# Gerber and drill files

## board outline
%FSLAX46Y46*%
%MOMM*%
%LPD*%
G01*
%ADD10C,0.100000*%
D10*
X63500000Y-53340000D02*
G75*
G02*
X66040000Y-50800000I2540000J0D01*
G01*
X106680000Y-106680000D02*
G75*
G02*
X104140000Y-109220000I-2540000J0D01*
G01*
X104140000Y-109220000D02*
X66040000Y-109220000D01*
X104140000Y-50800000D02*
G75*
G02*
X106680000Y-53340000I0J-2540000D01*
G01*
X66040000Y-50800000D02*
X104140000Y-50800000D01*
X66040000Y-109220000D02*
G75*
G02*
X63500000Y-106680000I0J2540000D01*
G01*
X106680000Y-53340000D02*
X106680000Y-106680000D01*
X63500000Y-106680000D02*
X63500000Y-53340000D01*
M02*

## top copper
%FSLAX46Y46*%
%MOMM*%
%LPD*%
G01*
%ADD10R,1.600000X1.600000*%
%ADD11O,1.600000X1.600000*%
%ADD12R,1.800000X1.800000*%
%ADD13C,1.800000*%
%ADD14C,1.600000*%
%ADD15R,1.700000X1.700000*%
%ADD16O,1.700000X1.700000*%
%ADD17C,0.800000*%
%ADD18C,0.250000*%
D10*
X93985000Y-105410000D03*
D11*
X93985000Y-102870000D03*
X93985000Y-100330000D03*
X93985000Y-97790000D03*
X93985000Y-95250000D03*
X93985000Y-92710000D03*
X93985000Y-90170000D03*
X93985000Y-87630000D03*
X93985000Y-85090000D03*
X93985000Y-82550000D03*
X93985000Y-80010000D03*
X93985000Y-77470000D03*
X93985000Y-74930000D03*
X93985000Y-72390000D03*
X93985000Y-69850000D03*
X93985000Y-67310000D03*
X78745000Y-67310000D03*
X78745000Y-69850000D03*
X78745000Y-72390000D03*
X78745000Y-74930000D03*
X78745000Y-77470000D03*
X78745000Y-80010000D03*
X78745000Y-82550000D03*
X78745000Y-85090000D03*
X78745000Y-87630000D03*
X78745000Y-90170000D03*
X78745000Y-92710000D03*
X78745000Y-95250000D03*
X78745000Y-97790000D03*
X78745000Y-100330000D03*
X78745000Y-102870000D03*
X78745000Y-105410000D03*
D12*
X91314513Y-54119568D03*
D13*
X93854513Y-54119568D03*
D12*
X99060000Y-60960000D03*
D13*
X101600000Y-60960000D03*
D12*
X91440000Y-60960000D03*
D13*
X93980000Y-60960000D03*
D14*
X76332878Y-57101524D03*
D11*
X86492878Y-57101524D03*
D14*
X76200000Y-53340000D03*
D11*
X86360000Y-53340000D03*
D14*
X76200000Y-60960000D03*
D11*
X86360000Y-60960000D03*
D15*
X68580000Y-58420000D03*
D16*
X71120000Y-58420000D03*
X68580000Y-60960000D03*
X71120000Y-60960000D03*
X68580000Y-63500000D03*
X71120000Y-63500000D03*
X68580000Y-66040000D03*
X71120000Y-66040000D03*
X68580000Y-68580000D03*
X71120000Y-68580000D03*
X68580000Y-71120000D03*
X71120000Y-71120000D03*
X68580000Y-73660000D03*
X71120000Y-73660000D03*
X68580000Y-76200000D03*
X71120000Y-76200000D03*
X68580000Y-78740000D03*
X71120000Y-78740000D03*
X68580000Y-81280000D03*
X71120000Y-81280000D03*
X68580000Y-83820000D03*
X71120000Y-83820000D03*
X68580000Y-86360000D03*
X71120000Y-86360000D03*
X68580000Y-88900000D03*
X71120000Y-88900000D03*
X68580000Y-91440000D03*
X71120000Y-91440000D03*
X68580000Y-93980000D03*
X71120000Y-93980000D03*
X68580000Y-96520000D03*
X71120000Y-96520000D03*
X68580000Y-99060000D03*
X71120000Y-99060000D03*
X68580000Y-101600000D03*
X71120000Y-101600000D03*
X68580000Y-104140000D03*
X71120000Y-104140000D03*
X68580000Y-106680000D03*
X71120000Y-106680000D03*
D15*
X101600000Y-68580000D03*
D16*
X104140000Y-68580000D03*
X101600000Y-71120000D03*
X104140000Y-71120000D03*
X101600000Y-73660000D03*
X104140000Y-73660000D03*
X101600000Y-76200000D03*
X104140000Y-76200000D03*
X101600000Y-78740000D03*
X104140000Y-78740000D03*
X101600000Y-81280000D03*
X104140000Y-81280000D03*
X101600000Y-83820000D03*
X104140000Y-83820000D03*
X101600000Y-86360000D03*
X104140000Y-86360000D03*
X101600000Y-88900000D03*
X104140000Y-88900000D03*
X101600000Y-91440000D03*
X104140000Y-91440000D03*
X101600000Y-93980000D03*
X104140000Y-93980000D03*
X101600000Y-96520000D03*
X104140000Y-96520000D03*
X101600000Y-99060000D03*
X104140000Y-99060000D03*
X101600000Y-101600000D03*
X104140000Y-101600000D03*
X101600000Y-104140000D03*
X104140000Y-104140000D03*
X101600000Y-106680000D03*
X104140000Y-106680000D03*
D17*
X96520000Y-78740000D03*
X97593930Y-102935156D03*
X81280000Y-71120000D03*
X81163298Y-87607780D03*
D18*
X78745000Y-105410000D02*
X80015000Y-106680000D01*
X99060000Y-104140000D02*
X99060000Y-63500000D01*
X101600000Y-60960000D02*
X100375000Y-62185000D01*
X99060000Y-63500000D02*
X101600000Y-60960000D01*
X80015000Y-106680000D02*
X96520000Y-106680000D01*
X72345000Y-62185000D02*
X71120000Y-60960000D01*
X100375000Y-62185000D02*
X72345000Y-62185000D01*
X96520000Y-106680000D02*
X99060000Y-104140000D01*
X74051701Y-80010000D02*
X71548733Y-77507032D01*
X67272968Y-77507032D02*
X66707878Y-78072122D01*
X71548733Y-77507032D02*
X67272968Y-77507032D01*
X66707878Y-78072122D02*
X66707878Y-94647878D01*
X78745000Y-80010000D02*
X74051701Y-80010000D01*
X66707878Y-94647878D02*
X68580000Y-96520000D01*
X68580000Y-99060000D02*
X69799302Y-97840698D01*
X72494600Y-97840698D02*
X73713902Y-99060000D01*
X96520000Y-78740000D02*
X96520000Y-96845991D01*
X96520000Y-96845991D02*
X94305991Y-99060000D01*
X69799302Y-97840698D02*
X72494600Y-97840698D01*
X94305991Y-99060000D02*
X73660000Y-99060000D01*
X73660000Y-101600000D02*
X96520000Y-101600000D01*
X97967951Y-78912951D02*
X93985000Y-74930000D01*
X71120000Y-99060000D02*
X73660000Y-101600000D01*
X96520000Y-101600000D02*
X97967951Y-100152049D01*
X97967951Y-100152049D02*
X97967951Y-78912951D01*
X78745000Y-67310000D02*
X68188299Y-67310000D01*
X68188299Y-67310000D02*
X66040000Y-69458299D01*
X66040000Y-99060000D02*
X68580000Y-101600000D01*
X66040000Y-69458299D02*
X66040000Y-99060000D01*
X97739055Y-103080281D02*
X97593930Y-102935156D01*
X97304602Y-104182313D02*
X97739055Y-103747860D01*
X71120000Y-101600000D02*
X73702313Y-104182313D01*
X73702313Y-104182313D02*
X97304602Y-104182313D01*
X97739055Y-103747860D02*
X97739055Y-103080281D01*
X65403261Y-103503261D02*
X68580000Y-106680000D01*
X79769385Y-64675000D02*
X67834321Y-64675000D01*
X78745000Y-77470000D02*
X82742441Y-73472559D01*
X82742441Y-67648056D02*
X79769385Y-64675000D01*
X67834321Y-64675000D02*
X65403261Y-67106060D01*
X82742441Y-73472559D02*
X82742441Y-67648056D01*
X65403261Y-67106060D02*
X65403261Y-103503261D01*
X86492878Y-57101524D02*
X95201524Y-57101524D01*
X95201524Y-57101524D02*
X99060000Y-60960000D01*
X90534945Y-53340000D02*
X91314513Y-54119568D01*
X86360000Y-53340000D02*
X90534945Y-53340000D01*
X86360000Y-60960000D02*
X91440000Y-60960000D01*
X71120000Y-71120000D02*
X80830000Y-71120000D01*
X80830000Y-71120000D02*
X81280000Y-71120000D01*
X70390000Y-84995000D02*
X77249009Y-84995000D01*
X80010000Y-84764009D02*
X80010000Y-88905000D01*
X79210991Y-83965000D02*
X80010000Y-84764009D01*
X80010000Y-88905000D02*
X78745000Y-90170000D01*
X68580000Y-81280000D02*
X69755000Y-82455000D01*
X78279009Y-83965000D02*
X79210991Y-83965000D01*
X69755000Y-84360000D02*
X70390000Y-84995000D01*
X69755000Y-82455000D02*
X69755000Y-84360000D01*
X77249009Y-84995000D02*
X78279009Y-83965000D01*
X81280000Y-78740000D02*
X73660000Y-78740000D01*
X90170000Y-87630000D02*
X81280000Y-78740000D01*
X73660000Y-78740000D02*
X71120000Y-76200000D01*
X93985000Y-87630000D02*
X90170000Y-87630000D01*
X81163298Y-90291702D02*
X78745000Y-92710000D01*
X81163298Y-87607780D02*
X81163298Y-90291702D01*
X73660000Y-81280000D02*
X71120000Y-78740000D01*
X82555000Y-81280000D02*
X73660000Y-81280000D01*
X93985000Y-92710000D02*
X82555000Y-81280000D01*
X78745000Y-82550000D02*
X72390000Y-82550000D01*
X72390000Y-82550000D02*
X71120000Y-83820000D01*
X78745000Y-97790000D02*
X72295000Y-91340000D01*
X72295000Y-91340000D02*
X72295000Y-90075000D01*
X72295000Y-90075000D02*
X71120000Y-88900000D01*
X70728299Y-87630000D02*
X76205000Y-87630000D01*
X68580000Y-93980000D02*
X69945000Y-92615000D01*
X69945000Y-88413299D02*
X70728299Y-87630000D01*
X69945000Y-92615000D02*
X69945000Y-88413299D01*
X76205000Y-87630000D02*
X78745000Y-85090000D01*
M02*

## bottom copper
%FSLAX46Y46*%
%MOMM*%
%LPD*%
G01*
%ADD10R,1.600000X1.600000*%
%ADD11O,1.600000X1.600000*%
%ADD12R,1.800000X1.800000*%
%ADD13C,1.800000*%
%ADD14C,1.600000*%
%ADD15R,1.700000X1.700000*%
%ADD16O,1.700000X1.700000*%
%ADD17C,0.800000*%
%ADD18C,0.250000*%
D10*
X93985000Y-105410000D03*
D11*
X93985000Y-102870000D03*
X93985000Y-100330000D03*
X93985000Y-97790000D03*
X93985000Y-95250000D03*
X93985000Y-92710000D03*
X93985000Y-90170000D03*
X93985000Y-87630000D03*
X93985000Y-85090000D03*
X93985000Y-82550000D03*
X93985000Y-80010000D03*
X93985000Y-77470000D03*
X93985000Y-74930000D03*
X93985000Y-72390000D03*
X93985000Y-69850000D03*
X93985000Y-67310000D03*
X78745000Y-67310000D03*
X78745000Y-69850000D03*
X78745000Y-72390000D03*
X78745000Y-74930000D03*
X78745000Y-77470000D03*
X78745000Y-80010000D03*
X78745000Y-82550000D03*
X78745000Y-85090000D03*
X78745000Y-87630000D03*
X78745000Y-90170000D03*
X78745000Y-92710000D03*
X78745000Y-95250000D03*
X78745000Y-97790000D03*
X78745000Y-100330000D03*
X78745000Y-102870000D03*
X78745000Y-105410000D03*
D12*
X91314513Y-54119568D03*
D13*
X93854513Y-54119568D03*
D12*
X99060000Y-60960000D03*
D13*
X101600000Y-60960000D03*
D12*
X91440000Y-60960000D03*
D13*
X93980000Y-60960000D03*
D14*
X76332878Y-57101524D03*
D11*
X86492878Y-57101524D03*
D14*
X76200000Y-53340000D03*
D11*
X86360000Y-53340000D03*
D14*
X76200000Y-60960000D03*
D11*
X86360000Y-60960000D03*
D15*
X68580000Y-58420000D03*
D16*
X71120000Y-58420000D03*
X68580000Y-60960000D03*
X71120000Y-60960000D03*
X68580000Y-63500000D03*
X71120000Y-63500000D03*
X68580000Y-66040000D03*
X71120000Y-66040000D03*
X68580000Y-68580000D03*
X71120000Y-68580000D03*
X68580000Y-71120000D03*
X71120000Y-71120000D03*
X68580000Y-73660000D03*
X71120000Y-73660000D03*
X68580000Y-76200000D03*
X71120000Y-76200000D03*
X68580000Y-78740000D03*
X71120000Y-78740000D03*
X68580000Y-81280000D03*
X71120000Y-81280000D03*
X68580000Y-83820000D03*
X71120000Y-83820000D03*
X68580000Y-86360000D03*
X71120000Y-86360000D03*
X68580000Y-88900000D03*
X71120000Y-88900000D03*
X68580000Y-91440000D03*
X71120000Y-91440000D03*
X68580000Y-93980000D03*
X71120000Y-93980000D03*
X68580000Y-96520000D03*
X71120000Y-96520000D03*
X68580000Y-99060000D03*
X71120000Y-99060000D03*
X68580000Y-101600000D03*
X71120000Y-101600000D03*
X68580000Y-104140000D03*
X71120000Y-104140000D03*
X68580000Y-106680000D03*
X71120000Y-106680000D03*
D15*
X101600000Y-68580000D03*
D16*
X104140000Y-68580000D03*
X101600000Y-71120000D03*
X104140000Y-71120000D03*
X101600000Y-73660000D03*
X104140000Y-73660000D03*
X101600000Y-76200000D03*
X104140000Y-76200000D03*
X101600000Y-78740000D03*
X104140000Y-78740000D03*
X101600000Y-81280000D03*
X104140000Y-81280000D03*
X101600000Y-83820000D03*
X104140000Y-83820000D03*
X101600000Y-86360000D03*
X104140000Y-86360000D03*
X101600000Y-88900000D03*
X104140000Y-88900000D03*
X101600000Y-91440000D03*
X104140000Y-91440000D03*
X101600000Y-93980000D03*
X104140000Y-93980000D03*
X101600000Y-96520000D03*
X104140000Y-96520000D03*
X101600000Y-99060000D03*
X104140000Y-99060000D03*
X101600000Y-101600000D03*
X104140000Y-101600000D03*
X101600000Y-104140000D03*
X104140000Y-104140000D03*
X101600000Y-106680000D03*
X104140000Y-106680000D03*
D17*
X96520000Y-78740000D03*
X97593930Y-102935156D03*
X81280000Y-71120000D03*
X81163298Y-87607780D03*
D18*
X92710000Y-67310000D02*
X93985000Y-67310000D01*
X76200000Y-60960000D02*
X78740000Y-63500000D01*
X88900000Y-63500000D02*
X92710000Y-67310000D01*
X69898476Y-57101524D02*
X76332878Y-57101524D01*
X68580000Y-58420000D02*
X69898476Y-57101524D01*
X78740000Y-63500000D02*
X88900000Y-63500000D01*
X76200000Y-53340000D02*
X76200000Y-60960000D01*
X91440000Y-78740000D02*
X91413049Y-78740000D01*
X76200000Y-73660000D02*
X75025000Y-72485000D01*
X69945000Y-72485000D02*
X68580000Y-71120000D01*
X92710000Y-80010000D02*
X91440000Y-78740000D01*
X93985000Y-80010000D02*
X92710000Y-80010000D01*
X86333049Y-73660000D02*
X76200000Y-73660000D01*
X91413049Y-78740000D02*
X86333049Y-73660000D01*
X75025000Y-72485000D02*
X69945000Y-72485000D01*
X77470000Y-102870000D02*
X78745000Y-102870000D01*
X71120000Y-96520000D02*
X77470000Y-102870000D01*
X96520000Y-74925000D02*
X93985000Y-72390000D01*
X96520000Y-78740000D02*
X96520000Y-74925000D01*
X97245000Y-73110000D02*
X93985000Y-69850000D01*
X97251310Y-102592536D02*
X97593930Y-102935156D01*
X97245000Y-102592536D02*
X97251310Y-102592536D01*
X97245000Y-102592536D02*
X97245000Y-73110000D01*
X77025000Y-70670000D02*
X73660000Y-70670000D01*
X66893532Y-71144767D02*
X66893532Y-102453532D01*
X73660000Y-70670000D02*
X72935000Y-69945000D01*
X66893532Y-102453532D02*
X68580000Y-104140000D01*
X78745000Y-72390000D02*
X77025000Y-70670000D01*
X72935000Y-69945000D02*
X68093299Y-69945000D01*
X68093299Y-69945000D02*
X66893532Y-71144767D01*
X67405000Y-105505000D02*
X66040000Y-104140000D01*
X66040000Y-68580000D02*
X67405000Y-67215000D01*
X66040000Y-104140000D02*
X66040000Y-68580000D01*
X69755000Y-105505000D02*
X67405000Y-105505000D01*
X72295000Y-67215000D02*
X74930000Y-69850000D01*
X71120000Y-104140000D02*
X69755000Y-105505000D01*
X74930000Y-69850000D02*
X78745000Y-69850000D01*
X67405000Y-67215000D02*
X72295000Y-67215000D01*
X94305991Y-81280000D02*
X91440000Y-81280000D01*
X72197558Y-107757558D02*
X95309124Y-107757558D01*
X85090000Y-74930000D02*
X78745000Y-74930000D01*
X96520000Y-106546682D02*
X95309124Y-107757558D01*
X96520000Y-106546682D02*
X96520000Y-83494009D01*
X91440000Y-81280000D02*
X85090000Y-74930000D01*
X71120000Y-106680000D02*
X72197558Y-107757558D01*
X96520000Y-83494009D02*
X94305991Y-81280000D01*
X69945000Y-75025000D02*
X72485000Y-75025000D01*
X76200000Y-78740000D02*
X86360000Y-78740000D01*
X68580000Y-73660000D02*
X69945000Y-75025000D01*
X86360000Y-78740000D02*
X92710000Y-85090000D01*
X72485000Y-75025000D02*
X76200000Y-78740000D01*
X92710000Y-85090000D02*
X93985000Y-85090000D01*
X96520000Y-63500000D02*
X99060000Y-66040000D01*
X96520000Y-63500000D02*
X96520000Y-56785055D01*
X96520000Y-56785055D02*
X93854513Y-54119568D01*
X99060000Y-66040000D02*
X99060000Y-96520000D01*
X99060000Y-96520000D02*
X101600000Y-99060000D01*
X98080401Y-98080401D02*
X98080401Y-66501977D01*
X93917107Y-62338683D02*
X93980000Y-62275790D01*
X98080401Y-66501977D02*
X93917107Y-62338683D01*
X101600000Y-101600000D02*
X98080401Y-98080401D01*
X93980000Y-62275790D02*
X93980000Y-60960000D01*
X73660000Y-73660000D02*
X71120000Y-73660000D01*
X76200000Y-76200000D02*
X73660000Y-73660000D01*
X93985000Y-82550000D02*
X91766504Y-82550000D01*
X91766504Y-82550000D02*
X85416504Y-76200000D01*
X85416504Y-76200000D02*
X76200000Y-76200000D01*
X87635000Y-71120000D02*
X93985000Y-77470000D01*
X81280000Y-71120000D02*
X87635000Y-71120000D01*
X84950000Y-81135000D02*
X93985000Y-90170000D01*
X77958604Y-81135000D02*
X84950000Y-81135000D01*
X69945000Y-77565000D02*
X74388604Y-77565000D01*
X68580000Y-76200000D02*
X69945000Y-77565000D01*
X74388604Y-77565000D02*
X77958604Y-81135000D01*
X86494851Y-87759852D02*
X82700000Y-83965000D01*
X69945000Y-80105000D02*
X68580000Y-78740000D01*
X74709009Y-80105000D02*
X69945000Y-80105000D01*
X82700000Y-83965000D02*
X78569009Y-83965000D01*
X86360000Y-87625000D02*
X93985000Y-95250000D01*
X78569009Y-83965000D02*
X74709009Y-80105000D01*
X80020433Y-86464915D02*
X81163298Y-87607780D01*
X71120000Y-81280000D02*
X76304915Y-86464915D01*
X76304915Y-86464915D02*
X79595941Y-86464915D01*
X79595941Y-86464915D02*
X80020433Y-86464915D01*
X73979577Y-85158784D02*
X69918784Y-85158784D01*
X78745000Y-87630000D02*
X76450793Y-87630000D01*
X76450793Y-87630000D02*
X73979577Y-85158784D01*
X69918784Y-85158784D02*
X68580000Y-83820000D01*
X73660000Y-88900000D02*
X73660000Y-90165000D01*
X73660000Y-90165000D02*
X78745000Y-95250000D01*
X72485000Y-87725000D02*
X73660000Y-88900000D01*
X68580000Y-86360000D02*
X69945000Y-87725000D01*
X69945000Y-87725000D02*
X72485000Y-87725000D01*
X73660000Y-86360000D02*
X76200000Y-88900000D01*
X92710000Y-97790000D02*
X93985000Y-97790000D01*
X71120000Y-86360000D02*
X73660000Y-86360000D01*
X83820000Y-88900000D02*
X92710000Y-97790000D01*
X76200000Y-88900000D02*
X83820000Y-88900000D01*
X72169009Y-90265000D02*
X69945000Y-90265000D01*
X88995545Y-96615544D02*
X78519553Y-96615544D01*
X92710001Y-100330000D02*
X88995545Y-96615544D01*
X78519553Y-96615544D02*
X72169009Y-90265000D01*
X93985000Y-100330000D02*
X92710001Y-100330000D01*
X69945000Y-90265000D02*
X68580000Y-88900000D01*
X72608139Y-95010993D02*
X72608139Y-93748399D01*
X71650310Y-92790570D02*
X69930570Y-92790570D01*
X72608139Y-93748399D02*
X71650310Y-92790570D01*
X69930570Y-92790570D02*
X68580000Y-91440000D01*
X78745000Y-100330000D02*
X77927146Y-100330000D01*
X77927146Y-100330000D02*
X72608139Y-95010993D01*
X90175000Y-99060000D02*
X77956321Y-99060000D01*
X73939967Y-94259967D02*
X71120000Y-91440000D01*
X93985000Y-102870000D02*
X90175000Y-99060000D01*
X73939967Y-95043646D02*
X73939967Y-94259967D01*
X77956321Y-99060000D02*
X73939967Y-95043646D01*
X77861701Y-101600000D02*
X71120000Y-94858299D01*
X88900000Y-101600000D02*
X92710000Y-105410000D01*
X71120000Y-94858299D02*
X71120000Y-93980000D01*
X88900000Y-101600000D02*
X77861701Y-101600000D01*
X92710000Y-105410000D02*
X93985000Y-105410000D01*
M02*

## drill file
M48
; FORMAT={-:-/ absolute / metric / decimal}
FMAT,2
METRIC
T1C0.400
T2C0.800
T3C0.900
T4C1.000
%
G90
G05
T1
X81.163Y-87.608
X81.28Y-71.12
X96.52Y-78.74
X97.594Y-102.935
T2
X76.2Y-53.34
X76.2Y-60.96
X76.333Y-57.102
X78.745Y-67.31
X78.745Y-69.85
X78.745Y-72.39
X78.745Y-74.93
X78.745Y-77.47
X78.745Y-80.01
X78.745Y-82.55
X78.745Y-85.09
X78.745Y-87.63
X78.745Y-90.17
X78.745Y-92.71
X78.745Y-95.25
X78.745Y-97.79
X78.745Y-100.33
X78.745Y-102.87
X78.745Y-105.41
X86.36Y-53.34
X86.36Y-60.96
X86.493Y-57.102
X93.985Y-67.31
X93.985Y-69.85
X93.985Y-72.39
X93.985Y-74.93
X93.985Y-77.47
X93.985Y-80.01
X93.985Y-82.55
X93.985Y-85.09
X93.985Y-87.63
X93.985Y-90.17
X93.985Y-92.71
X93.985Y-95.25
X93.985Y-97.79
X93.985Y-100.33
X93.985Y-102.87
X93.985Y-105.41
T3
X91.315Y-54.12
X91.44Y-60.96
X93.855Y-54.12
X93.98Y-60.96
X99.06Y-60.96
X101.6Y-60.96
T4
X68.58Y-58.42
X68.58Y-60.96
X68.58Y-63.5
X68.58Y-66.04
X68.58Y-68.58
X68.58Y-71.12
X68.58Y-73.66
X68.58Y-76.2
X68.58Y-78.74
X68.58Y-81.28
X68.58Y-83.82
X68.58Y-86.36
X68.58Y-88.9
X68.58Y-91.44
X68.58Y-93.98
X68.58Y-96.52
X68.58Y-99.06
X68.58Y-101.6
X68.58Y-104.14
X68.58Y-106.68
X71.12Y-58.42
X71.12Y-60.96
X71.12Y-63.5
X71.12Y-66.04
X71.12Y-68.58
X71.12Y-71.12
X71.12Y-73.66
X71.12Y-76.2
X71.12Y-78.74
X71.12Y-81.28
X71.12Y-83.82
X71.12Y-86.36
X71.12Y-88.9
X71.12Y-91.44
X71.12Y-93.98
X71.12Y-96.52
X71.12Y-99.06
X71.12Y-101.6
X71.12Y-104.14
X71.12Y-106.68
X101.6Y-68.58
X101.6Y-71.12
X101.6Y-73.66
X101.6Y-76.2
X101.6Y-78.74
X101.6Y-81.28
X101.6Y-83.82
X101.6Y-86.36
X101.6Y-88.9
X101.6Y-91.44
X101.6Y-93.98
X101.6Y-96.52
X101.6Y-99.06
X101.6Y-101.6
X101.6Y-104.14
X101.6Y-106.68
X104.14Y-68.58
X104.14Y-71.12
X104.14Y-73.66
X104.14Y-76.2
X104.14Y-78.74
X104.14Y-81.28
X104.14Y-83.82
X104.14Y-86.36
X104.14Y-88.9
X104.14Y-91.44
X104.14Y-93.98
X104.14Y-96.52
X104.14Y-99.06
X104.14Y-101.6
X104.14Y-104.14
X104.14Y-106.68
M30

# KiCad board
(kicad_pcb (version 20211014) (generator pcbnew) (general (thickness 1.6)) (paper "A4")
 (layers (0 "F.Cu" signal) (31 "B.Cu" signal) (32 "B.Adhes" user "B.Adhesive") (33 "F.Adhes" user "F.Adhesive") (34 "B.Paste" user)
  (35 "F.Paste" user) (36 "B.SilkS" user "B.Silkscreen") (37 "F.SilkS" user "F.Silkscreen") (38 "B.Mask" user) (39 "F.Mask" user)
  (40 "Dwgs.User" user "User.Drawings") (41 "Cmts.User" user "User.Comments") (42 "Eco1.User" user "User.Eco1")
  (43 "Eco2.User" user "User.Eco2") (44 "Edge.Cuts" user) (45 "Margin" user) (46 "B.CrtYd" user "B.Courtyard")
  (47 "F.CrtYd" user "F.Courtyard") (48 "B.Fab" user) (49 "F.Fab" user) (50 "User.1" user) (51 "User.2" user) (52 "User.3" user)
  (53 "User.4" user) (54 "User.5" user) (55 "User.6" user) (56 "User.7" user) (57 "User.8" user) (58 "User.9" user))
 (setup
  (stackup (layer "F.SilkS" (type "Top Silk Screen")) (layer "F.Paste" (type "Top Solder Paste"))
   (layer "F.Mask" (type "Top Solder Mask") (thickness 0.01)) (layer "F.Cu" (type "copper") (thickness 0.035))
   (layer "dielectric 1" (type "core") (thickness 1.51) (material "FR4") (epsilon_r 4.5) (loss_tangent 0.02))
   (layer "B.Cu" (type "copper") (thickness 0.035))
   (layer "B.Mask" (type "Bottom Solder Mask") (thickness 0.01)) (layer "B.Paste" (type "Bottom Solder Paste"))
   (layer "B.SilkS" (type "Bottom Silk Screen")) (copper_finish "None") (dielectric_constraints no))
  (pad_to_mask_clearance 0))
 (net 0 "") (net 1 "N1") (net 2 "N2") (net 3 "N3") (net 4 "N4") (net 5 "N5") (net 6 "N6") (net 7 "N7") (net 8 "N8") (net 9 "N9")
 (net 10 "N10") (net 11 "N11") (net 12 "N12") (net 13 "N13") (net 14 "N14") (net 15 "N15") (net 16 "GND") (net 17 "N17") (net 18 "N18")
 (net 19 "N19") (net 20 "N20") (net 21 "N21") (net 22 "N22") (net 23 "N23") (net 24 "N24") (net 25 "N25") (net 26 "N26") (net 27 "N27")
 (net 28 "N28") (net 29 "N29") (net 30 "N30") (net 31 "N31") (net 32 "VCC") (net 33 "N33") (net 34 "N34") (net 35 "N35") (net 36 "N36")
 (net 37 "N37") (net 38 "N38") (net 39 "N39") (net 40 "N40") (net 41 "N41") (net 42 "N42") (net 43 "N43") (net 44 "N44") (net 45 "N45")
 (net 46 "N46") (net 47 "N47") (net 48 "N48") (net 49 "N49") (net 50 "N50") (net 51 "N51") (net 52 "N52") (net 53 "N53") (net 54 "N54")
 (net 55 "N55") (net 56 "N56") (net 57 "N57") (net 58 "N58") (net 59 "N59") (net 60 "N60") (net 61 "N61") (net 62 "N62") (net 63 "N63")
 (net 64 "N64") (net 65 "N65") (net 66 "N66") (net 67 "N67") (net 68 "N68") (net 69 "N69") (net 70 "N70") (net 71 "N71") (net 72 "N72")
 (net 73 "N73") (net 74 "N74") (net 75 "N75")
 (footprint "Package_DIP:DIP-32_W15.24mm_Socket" (layer "F.Cu") (at 93.985 105.41 180)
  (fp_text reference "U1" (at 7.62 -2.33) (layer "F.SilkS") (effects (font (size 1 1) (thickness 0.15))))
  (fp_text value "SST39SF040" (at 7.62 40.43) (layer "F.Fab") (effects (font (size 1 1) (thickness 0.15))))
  (pad "1" thru_hole rect (at 0 0 180) (size 1.6 1.6) (drill 0.8) (layers *.Cu *.Mask) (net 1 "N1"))
  (pad "2" thru_hole oval (at 0 2.54 180) (size 1.6 1.6) (drill 0.8) (layers *.Cu *.Mask) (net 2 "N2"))
  (pad "3" thru_hole oval (at 0 5.08 180) (size 1.6 1.6) (drill 0.8) (layers *.Cu *.Mask) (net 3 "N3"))
  (pad "4" thru_hole oval (at 0 7.62 180) (size 1.6 1.6) (drill 0.8) (layers *.Cu *.Mask) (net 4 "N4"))
  (pad "5" thru_hole oval (at 0 10.16 180) (size 1.6 1.6) (drill 0.8) (layers *.Cu *.Mask) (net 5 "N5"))
  (pad "6" thru_hole oval (at 0 12.7 180) (size 1.6 1.6) (drill 0.8) (layers *.Cu *.Mask) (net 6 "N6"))
  (pad "7" thru_hole oval (at 0 15.24 180) (size 1.6 1.6) (drill 0.8) (layers *.Cu *.Mask) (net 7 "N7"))
  (pad "8" thru_hole oval (at 0 17.78 180) (size 1.6 1.6) (drill 0.8) (layers *.Cu *.Mask) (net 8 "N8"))
  (pad "9" thru_hole oval (at 0 20.32 180) (size 1.6 1.6) (drill 0.8) (layers *.Cu *.Mask) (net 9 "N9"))
  (pad "10" thru_hole oval (at 0 22.86 180) (size 1.6 1.6) (drill 0.8) (layers *.Cu *.Mask) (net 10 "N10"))
  (pad "11" thru_hole oval (at 0 25.4 180) (size 1.6 1.6) (drill 0.8) (layers *.Cu *.Mask) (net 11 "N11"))
  (pad "12" thru_hole oval (at 0 27.94 180) (size 1.6 1.6) (drill 0.8) (layers *.Cu *.Mask) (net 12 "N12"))
  (pad "13" thru_hole oval (at 0 30.48 180) (size 1.6 1.6) (drill 0.8) (layers *.Cu *.Mask) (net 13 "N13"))
  (pad "14" thru_hole oval (at 0 33.02 180) (size 1.6 1.6) (drill 0.8) (layers *.Cu *.Mask) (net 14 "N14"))
  (pad "15" thru_hole oval (at 0 35.56 180) (size 1.6 1.6) (drill 0.8) (layers *.Cu *.Mask) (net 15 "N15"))
  (pad "16" thru_hole oval (at 0 38.1 180) (size 1.6 1.6) (drill 0.8) (layers *.Cu *.Mask) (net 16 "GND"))
  (pad "17" thru_hole oval (at 15.24 38.1 180) (size 1.6 1.6) (drill 0.8) (layers *.Cu *.Mask) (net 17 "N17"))
  (pad "18" thru_hole oval (at 15.24 35.56 180) (size 1.6 1.6) (drill 0.8) (layers *.Cu *.Mask) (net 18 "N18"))
  (pad "19" thru_hole oval (at 15.24 33.02 180) (size 1.6 1.6) (drill 0.8) (layers *.Cu *.Mask) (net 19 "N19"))
  (pad "20" thru_hole oval (at 15.24 30.48 180) (size 1.6 1.6) (drill 0.8) (layers *.Cu *.Mask) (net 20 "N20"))
  (pad "21" thru_hole oval (at 15.24 27.94 180) (size 1.6 1.6) (drill 0.8) (layers *.Cu *.Mask) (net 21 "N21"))
  (pad "22" thru_hole oval (at 15.24 25.4 180) (size 1.6 1.6) (drill 0.8) (layers *.Cu *.Mask) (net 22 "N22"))
  (pad "23" thru_hole oval (at 15.24 22.86 180) (size 1.6 1.6) (drill 0.8) (layers *.Cu *.Mask) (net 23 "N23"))
  (pad "24" thru_hole oval (at 15.24 20.32 180) (size 1.6 1.6) (drill 0.8) (layers *.Cu *.Mask) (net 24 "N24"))
  (pad "25" thru_hole oval (at 15.24 17.78 180) (size 1.6 1.6) (drill 0.8) (layers *.Cu *.Mask) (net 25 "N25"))
  (pad "26" thru_hole oval (at 15.24 15.24 180) (size 1.6 1.6) (drill 0.8) (layers *.Cu *.Mask) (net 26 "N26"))
  (pad "27" thru_hole oval (at 15.24 12.7 180) (size 1.6 1.6) (drill 0.8) (layers *.Cu *.Mask) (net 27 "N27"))
  (pad "28" thru_hole oval (at 15.24 10.16 180) (size 1.6 1.6) (drill 0.8) (layers *.Cu *.Mask) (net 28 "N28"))
  (pad "29" thru_hole oval (at 15.24 7.62 180) (size 1.6 1.6) (drill 0.8) (layers *.Cu *.Mask) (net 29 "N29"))
  (pad "30" thru_hole oval (at 15.24 5.08 180) (size 1.6 1.6) (drill 0.8) (layers *.Cu *.Mask) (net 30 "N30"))
  (pad "31" thru_hole oval (at 15.24 2.54 180) (size 1.6 1.6) (drill 0.8) (layers *.Cu *.Mask) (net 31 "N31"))
  (pad "32" thru_hole oval (at 15.24 0 180) (size 1.6 1.6) (drill 0.8) (layers *.Cu *.Mask) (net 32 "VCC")))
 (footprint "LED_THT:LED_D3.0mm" (layer "F.Cu") (at 91.314513 54.119568)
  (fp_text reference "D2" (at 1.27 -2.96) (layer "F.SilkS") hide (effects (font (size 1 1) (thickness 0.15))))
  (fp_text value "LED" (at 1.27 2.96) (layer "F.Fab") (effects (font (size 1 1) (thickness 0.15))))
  (pad "1" thru_hole rect (at 0 0) (size 1.8 1.8) (drill 0.9) (layers *.Cu *.Mask) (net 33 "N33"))
  (pad "2" thru_hole circle (at 2.54 0) (size 1.8 1.8) (drill 0.9) (layers *.Cu *.Mask) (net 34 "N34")))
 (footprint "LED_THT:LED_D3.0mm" (layer "F.Cu") (at 99.06 60.96)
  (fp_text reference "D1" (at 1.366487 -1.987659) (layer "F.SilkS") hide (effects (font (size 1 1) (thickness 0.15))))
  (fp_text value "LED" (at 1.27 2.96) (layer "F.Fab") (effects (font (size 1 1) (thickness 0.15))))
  (pad "1" thru_hole rect (at 0 0) (size 1.8 1.8) (drill 0.9) (layers *.Cu *.Mask) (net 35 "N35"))
  (pad "2" thru_hole circle (at 2.54 0) (size 1.8 1.8) (drill 0.9) (layers *.Cu *.Mask) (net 32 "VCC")))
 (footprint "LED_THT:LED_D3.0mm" (layer "F.Cu") (at 91.44 60.96)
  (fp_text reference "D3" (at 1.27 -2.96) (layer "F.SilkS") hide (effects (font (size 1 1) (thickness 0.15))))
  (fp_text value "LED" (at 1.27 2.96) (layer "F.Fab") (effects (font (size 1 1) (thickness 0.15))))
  (pad "1" thru_hole rect (at 0 0) (size 1.8 1.8) (drill 0.9) (layers *.Cu *.Mask) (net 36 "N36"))
  (pad "2" thru_hole circle (at 2.54 0) (size 1.8 1.8) (drill 0.9) (layers *.Cu *.Mask) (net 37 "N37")))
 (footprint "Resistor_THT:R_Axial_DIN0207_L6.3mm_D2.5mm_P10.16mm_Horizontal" (layer "F.Cu") (at 76.332878 57.101524)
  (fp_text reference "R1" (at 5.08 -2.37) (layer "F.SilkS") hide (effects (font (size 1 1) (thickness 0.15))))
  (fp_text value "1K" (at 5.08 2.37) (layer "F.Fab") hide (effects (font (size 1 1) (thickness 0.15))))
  (pad "1" thru_hole circle (at 0 0) (size 1.6 1.6) (drill 0.8) (layers *.Cu *.Mask) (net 16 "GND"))
  (pad "2" thru_hole oval (at 10.16 0) (size 1.6 1.6) (drill 0.8) (layers *.Cu *.Mask) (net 35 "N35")))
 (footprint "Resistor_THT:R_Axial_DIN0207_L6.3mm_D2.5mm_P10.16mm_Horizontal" (layer "F.Cu") (at 76.2 53.34)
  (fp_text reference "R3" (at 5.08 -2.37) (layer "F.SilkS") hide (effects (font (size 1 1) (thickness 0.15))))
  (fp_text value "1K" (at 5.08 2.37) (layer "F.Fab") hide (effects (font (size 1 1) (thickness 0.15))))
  (pad "1" thru_hole circle (at 0 0) (size 1.6 1.6) (drill 0.8) (layers *.Cu *.Mask) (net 16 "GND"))
  (pad "2" thru_hole oval (at 10.16 0) (size 1.6 1.6) (drill 0.8) (layers *.Cu *.Mask) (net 33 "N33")))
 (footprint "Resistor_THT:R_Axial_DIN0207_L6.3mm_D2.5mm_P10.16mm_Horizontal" (layer "F.Cu") (at 76.2 60.96)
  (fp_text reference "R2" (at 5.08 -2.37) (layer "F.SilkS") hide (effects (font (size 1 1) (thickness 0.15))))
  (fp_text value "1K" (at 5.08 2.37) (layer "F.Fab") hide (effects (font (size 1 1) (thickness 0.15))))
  (pad "1" thru_hole circle (at 0 0) (size 1.6 1.6) (drill 0.8) (layers *.Cu *.Mask) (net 16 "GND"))
  (pad "2" thru_hole oval (at 10.16 0) (size 1.6 1.6) (drill 0.8) (layers *.Cu *.Mask) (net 36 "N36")))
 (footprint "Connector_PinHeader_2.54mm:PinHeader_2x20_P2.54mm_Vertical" (layer "F.Cu") (at 68.58 58.42)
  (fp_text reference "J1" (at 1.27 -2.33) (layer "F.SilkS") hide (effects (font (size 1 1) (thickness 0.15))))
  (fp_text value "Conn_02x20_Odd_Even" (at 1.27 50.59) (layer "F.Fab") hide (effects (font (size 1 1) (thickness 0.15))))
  (pad "1" thru_hole rect (at 0 0) (size 1.7 1.7) (drill 1) (layers *.Cu *.Mask) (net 16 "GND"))
  (pad "2" thru_hole oval (at 2.54 0) (size 1.7 1.7) (drill 1) (layers *.Cu *.Mask) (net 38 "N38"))
  (pad "3" thru_hole oval (at 0 2.54) (size 1.7 1.7) (drill 1) (layers *.Cu *.Mask) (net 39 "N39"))
  (pad "4" thru_hole oval (at 2.54 2.54) (size 1.7 1.7) (drill 1) (layers *.Cu *.Mask) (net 32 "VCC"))
  (pad "5" thru_hole oval (at 0 5.08) (size 1.7 1.7) (drill 1) (layers *.Cu *.Mask) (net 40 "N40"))
  (pad "6" thru_hole oval (at 2.54 5.08) (size 1.7 1.7) (drill 1) (layers *.Cu *.Mask) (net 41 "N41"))
  (pad "7" thru_hole oval (at 0 7.62) (size 1.7 1.7) (drill 1) (layers *.Cu *.Mask) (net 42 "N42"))
  (pad "8" thru_hole oval (at 2.54 7.62) (size 1.7 1.7) (drill 1) (layers *.Cu *.Mask) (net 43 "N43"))
  (pad "9" thru_hole oval (at 0 10.16) (size 1.7 1.7) (drill 1) (layers *.Cu *.Mask) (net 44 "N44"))
  (pad "10" thru_hole oval (at 2.54 10.16) (size 1.7 1.7) (drill 1) (layers *.Cu *.Mask) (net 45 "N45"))
  (pad "11" thru_hole oval (at 0 12.7) (size 1.7 1.7) (drill 1) (layers *.Cu *.Mask) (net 11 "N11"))
  (pad "12" thru_hole oval (at 2.54 12.7) (size 1.7 1.7) (drill 1) (layers *.Cu *.Mask) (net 12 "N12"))
  (pad "13" thru_hole oval (at 0 15.24) (size 1.7 1.7) (drill 1) (layers *.Cu *.Mask) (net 9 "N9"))
  (pad "14" thru_hole oval (at 2.54 15.24) (size 1.7 1.7) (drill 1) (layers *.Cu *.Mask) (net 10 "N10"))
  (pad "15" thru_hole oval (at 0 17.78) (size 1.7 1.7) (drill 1) (layers *.Cu *.Mask) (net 7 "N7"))
  (pad "16" thru_hole oval (at 2.54 17.78) (size 1.7 1.7) (drill 1) (layers *.Cu *.Mask) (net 8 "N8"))
  (pad "17" thru_hole oval (at 0 20.32) (size 1.7 1.7) (drill 1) (layers *.Cu *.Mask) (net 5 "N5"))
  (pad "18" thru_hole oval (at 2.54 20.32) (size 1.7 1.7) (drill 1) (layers *.Cu *.Mask) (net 6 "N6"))
  (pad "19" thru_hole oval (at 0 22.86) (size 1.7 1.7) (drill 1) (layers *.Cu *.Mask) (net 26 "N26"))
  (pad "20" thru_hole oval (at 2.54 22.86) (size 1.7 1.7) (drill 1) (layers *.Cu *.Mask) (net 27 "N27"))
  (pad "21" thru_hole oval (at 0 25.4) (size 1.7 1.7) (drill 1) (layers *.Cu *.Mask) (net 25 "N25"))
  (pad "22" thru_hole oval (at 2.54 25.4) (size 1.7 1.7) (drill 1) (layers *.Cu *.Mask) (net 23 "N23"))
  (pad "23" thru_hole oval (at 0 27.94) (size 1.7 1.7) (drill 1) (layers *.Cu *.Mask) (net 28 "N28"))
  (pad "24" thru_hole oval (at 2.54 27.94) (size 1.7 1.7) (drill 1) (layers *.Cu *.Mask) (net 4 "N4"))
  (pad "25" thru_hole oval (at 0 30.48) (size 1.7 1.7) (drill 1) (layers *.Cu *.Mask) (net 3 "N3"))
  (pad "26" thru_hole oval (at 2.54 30.48) (size 1.7 1.7) (drill 1) (layers *.Cu *.Mask) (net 29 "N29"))
  (pad "27" thru_hole oval (at 0 33.02) (size 1.7 1.7) (drill 1) (layers *.Cu *.Mask) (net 30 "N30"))
  (pad "28" thru_hole oval (at 2.54 33.02) (size 1.7 1.7) (drill 1) (layers *.Cu *.Mask) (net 2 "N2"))
  (pad "29" thru_hole oval (at 0 35.56) (size 1.7 1.7) (drill 1) (layers *.Cu *.Mask) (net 24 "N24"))
  (pad "30" thru_hole oval (at 2.54 35.56) (size 1.7 1.7) (drill 1) (layers *.Cu *.Mask) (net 1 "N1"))
  (pad "31" thru_hole oval (at 0 38.1) (size 1.7 1.7) (drill 1) (layers *.Cu *.Mask) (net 22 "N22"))
  (pad "32" thru_hole oval (at 2.54 38.1) (size 1.7 1.7) (drill 1) (layers *.Cu *.Mask) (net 31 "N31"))
  (pad "33" thru_hole oval (at 0 40.64) (size 1.7 1.7) (drill 1) (layers *.Cu *.Mask) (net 14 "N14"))
  (pad "34" thru_hole oval (at 2.54 40.64) (size 1.7 1.7) (drill 1) (layers *.Cu *.Mask) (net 13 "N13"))
  (pad "35" thru_hole oval (at 0 43.18) (size 1.7 1.7) (drill 1) (layers *.Cu *.Mask) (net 17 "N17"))
  (pad "36" thru_hole oval (at 2.54 43.18) (size 1.7 1.7) (drill 1) (layers *.Cu *.Mask) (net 15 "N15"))
  (pad "37" thru_hole oval (at 0 45.72) (size 1.7 1.7) (drill 1) (layers *.Cu *.Mask) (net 19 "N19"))
  (pad "38" thru_hole oval (at 2.54 45.72) (size 1.7 1.7) (drill 1) (layers *.Cu *.Mask) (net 18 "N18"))
  (pad "39" thru_hole oval (at 0 48.26) (size 1.7 1.7) (drill 1) (layers *.Cu *.Mask) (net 21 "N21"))
  (pad "40" thru_hole oval (at 2.54 48.26) (size 1.7 1.7) (drill 1) (layers *.Cu *.Mask) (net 20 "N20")))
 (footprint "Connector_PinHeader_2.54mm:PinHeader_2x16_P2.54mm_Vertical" (layer "F.Cu") (at 101.6 68.58)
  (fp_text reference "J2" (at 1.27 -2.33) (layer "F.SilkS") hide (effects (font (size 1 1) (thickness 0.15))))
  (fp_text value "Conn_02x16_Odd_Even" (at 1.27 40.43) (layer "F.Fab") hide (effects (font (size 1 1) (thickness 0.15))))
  (pad "1" thru_hole rect (at 0 0) (size 1.7 1.7) (drill 1) (layers *.Cu *.Mask) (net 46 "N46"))
  (pad "2" thru_hole oval (at 2.54 0) (size 1.7 1.7) (drill 1) (layers *.Cu *.Mask) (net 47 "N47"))
  (pad "3" thru_hole oval (at 0 2.54) (size 1.7 1.7) (drill 1) (layers *.Cu *.Mask) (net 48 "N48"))
  (pad "4" thru_hole oval (at 2.54 2.54) (size 1.7 1.7) (drill 1) (layers *.Cu *.Mask) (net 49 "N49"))
  (pad "5" thru_hole oval (at 0 5.08) (size 1.7 1.7) (drill 1) (layers *.Cu *.Mask) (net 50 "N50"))
  (pad "6" thru_hole oval (at 2.54 5.08) (size 1.7 1.7) (drill 1) (layers *.Cu *.Mask) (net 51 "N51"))
  (pad "7" thru_hole oval (at 0 7.62) (size 1.7 1.7) (drill 1) (layers *.Cu *.Mask) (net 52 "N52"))
  (pad "8" thru_hole oval (at 2.54 7.62) (size 1.7 1.7) (drill 1) (layers *.Cu *.Mask) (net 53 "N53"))
  (pad "9" thru_hole oval (at 0 10.16) (size 1.7 1.7) (drill 1) (layers *.Cu *.Mask) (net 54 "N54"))
  (pad "10" thru_hole oval (at 2.54 10.16) (size 1.7 1.7) (drill 1) (layers *.Cu *.Mask) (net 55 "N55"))
  (pad "11" thru_hole oval (at 0 12.7) (size 1.7 1.7) (drill 1) (layers *.Cu *.Mask) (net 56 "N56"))
  (pad "12" thru_hole oval (at 2.54 12.7) (size 1.7 1.7) (drill 1) (layers *.Cu *.Mask) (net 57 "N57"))
  (pad "13" thru_hole oval (at 0 15.24) (size 1.7 1.7) (drill 1) (layers *.Cu *.Mask) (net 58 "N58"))
  (pad "14" thru_hole oval (at 2.54 15.24) (size 1.7 1.7) (drill 1) (layers *.Cu *.Mask) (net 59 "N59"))
  (pad "15" thru_hole oval (at 0 17.78) (size 1.7 1.7) (drill 1) (layers *.Cu *.Mask) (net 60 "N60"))
  (pad "16" thru_hole oval (at 2.54 17.78) (size 1.7 1.7) (drill 1) (layers *.Cu *.Mask) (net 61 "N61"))
  (pad "17" thru_hole oval (at 0 20.32) (size 1.7 1.7) (drill 1) (layers *.Cu *.Mask) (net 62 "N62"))
  (pad "18" thru_hole oval (at 2.54 20.32) (size 1.7 1.7) (drill 1) (layers *.Cu *.Mask) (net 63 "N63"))
  (pad "19" thru_hole oval (at 0 22.86) (size 1.7 1.7) (drill 1) (layers *.Cu *.Mask) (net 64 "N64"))
  (pad "20" thru_hole oval (at 2.54 22.86) (size 1.7 1.7) (drill 1) (layers *.Cu *.Mask) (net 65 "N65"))
  (pad "21" thru_hole oval (at 0 25.4) (size 1.7 1.7) (drill 1) (layers *.Cu *.Mask) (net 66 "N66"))
  (pad "22" thru_hole oval (at 2.54 25.4) (size 1.7 1.7) (drill 1) (layers *.Cu *.Mask) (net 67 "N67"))
  (pad "23" thru_hole oval (at 0 27.94) (size 1.7 1.7) (drill 1) (layers *.Cu *.Mask) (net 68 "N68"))
  (pad "24" thru_hole oval (at 2.54 27.94) (size 1.7 1.7) (drill 1) (layers *.Cu *.Mask) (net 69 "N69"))
  (pad "25" thru_hole oval (at 0 30.48) (size 1.7 1.7) (drill 1) (layers *.Cu *.Mask) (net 34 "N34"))
  (pad "26" thru_hole oval (at 2.54 30.48) (size 1.7 1.7) (drill 1) (layers *.Cu *.Mask) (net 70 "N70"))
  (pad "27" thru_hole oval (at 0 33.02) (size 1.7 1.7) (drill 1) (layers *.Cu *.Mask) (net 37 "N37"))
  (pad "28" thru_hole oval (at 2.54 33.02) (size 1.7 1.7) (drill 1) (layers *.Cu *.Mask) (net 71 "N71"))
  (pad "29" thru_hole oval (at 0 35.56) (size 1.7 1.7) (drill 1) (layers *.Cu *.Mask) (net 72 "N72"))
  (pad "30" thru_hole oval (at 2.54 35.56) (size 1.7 1.7) (drill 1) (layers *.Cu *.Mask) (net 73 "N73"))
  (pad "31" thru_hole oval (at 0 38.1) (size 1.7 1.7) (drill 1) (layers *.Cu *.Mask) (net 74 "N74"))
  (pad "32" thru_hole oval (at 2.54 38.1) (size 1.7 1.7) (drill 1) (layers *.Cu *.Mask) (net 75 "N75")))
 (gr_arc (start 63.5 53.34) (mid 64.243949 51.543949) (end 66.04 50.8) (layer "Edge.Cuts") (width 0.1))
 (gr_arc (start 106.68 106.68) (mid 105.936051 108.476051) (end 104.14 109.22) (layer "Edge.Cuts") (width 0.1))
 (gr_line (start 104.14 109.22) (end 66.04 109.22) (layer "Edge.Cuts") (width 0.1))
 (gr_arc (start 104.14 50.8) (mid 105.936051 51.543949) (end 106.68 53.34) (layer "Edge.Cuts") (width 0.1))
 (gr_line (start 66.04 50.8) (end 104.14 50.8) (layer "Edge.Cuts") (width 0.1))
 (gr_arc (start 66.04 109.22) (mid 64.243949 108.476051) (end 63.5 106.68) (layer "Edge.Cuts") (width 0.1))
 (gr_line (start 106.68 53.34) (end 106.68 106.68) (layer "Edge.Cuts") (width 0.1))
 (gr_line (start 63.5 106.68) (end 63.5 53.34) (layer "Edge.Cuts") (width 0.1))
 (segment (start 92.71 67.31) (end 93.985 67.31) (width 0.25) (layer "B.Cu") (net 16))
 (segment (start 76.2 60.96) (end 78.74 63.5) (width 0.25) (layer "B.Cu") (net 16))
 (segment (start 88.9 63.5) (end 92.71 67.31) (width 0.25) (layer "B.Cu") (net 16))
 (segment (start 69.898476 57.101524) (end 76.332878 57.101524) (width 0.25) (layer "B.Cu") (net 16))
 (segment (start 68.58 58.42) (end 69.898476 57.101524) (width 0.25) (layer "B.Cu") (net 16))
 (segment (start 78.74 63.5) (end 88.9 63.5) (width 0.25) (layer "B.Cu") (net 16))
 (segment (start 76.2 53.34) (end 76.2 60.96) (width 0.25) (layer "B.Cu") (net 16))
 (segment (start 78.745 105.41) (end 80.015 106.68) (width 0.25) (layer "F.Cu") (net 32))
 (segment (start 99.06 104.14) (end 99.06 63.5) (width 0.25) (layer "F.Cu") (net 32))
 (segment (start 101.6 60.96) (end 100.375 62.185) (width 0.25) (layer "F.Cu") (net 32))
 (segment (start 99.06 63.5) (end 101.6 60.96) (width 0.25) (layer "F.Cu") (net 32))
 (segment (start 80.015 106.68) (end 96.52 106.68) (width 0.25) (layer "F.Cu") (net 32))
 (segment (start 72.345 62.185) (end 71.12 60.96) (width 0.25) (layer "F.Cu") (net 32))
 (segment (start 100.375 62.185) (end 72.345 62.185) (width 0.25) (layer "F.Cu") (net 32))
 (segment (start 96.52 106.68) (end 99.06 104.14) (width 0.25) (layer "F.Cu") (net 32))
 (segment (start 91.44 78.74) (end 91.413049 78.74) (width 0.25) (layer "B.Cu") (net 11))
 (segment (start 76.2 73.66) (end 75.025 72.485) (width 0.25) (layer "B.Cu") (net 11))
 (segment (start 69.945 72.485) (end 68.58 71.12) (width 0.25) (layer "B.Cu") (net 11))
 (segment (start 92.71 80.01) (end 91.44 78.74) (width 0.25) (layer "B.Cu") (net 11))
 (segment (start 93.985 80.01) (end 92.71 80.01) (width 0.25) (layer "B.Cu") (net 11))
 (segment (start 86.333049 73.66) (end 76.2 73.66) (width 0.25) (layer "B.Cu") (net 11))
 (segment (start 91.413049 78.74) (end 86.333049 73.66) (width 0.25) (layer "B.Cu") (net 11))
 (segment (start 75.025 72.485) (end 69.945 72.485) (width 0.25) (layer "B.Cu") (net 11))
 (segment (start 74.051701 80.01) (end 71.548733 77.507032) (width 0.25) (layer "F.Cu") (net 22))
 (segment (start 67.272968 77.507032) (end 66.707878 78.072122) (width 0.25) (layer "F.Cu") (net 22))
 (segment (start 71.548733 77.507032) (end 67.272968 77.507032) (width 0.25) (layer "F.Cu") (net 22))
 (segment (start 66.707878 78.072122) (end 66.707878 94.647878) (width 0.25) (layer "F.Cu") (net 22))
 (segment (start 78.745 80.01) (end 74.051701 80.01) (width 0.25) (layer "F.Cu") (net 22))
 (segment (start 66.707878 94.647878) (end 68.58 96.52) (width 0.25) (layer "F.Cu") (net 22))
 (segment (start 77.47 102.87) (end 78.745 102.87) (width 0.25) (layer "B.Cu") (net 31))
 (segment (start 71.12 96.52) (end 77.47 102.87) (width 0.25) (layer "B.Cu") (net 31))
 (segment (start 68.58 99.06) (end 69.799302 97.840698) (width 0.25) (layer "F.Cu") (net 14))
 (segment (start 72.4946 97.840698) (end 73.713902 99.06) (width 0.25) (layer "F.Cu") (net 14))
 (segment (start 96.52 78.74) (end 96.52 96.845991) (width 0.25) (layer "F.Cu") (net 14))
 (segment (start 96.52 96.845991) (end 94.305991 99.06) (width 0.25) (layer "F.Cu") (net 14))
 (segment (start 69.799302 97.840698) (end 72.4946 97.840698) (width 0.25) (layer "F.Cu") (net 14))
 (segment (start 94.305991 99.06) (end 73.66 99.06) (width 0.25) (layer "F.Cu") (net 14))
 (via (at 96.52 78.74) (size 0.8) (drill 0.4) (layers "F.Cu" "B.Cu") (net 14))
 (segment (start 96.52 74.925) (end 93.985 72.39) (width 0.25) (layer "B.Cu") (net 14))
 (segment (start 96.52 78.74) (end 96.52 74.925) (width 0.25) (layer "B.Cu") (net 14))
 (segment (start 73.66 101.6) (end 96.52 101.6) (width 0.25) (layer "F.Cu") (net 13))
 (segment (start 97.967951 78.912951) (end 93.985 74.93) (width 0.25) (layer "F.Cu") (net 13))
 (segment (start 71.12 99.06) (end 73.66 101.6) (width 0.25) (layer "F.Cu") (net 13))
 (segment (start 96.52 101.6) (end 97.967951 100.152049) (width 0.25) (layer "F.Cu") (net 13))
 (segment (start 97.967951 100.152049) (end 97.967951 78.912951) (width 0.25) (layer "F.Cu") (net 13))
 (segment (start 78.745 67.31) (end 68.188299 67.31) (width 0.25) (layer "F.Cu") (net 17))
 (segment (start 68.188299 67.31) (end 66.04 69.458299) (width 0.25) (layer "F.Cu") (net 17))
 (segment (start 66.04 99.06) (end 68.58 101.6) (width 0.25) (layer "F.Cu") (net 17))
 (segment (start 66.04 69.458299) (end 66.04 99.06) (width 0.25) (layer "F.Cu") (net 17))
 (segment (start 97.739055 103.080281) (end 97.59393 102.935156) (width 0.25) (layer "F.Cu") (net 15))
 (segment (start 97.304602 104.182313) (end 97.739055 103.74786) (width 0.25) (layer "F.Cu") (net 15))
 (segment (start 71.12 101.6) (end 73.702313 104.182313) (width 0.25) (layer "F.Cu") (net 15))
 (segment (start 73.702313 104.182313) (end 97.304602 104.182313) (width 0.25) (layer "F.Cu") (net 15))
 (segment (start 97.739055 103.74786) (end 97.739055 103.080281) (width 0.25) (layer "F.Cu") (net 15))
 (via (at 97.59393 102.935156) (size 0.8) (drill 0.4) (layers "F.Cu" "B.Cu") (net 15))
 (segment (start 97.245 73.11) (end 93.985 69.85) (width 0.25) (layer "B.Cu") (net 15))
 (segment (start 97.25131 102.592536) (end 97.59393 102.935156) (width 0.25) (layer "B.Cu") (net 15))
 (segment (start 97.245 102.592536) (end 97.25131 102.592536) (width 0.25) (layer "B.Cu") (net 15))
 (segment (start 97.245 102.592536) (end 97.245 73.11) (width 0.25) (layer "B.Cu") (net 15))
 (segment (start 77.025 70.67) (end 73.66 70.67) (width 0.25) (layer "B.Cu") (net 19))
 (segment (start 66.893532 71.144767) (end 66.893532 102.453532) (width 0.25) (layer "B.Cu") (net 19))
 (segment (start 73.66 70.67) (end 72.935 69.945) (width 0.25) (layer "B.Cu") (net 19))
 (segment (start 66.893532 102.453532) (end 68.58 104.14) (width 0.25) (layer "B.Cu") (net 19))
 (segment (start 78.745 72.39) (end 77.025 70.67) (width 0.25) (layer "B.Cu") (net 19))
 (segment (start 72.935 69.945) (end 68.093299 69.945) (width 0.25) (layer "B.Cu") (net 19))
 (segment (start 68.093299 69.945) (end 66.893532 71.144767) (width 0.25) (layer "B.Cu") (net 19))
 (segment (start 67.405 105.505) (end 66.04 104.14) (width 0.25) (layer "B.Cu") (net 18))
 (segment (start 66.04 68.58) (end 67.405 67.215) (width 0.25) (layer "B.Cu") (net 18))
 (segment (start 66.04 104.14) (end 66.04 68.58) (width 0.25) (layer "B.Cu") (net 18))
 (segment (start 69.755 105.505) (end 67.405 105.505) (width 0.25) (layer "B.Cu") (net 18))
 (segment (start 72.295 67.215) (end 74.93 69.85) (width 0.25) (layer "B.Cu") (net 18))
 (segment (start 71.12 104.14) (end 69.755 105.505) (width 0.25) (layer "B.Cu") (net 18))
 (segment (start 74.93 69.85) (end 78.745 69.85) (width 0.25) (layer "B.Cu") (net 18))
 (segment (start 67.405 67.215) (end 72.295 67.215) (width 0.25) (layer "B.Cu") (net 18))
 (segment (start 65.403261 103.503261) (end 68.58 106.68) (width 0.25) (layer "F.Cu") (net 21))
 (segment (start 79.769385 64.675) (end 67.834321 64.675) (width 0.25) (layer "F.Cu") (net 21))
 (segment (start 78.745 77.47) (end 82.742441 73.472559) (width 0.25) (layer "F.Cu") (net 21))
 (segment (start 82.742441 67.648056) (end 79.769385 64.675) (width 0.25) (layer "F.Cu") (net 21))
 (segment (start 67.834321 64.675) (end 65.403261 67.10606) (width 0.25) (layer "F.Cu") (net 21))
 (segment (start 82.742441 73.472559) (end 82.742441 67.648056) (width 0.25) (layer "F.Cu") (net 21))
 (segment (start 65.403261 67.10606) (end 65.403261 103.503261) (width 0.25) (layer "F.Cu") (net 21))
 (segment (start 94.305991 81.28) (end 91.44 81.28) (width 0.25) (layer "B.Cu") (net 20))
 (segment (start 72.197558 107.757558) (end 95.309124 107.757558) (width 0.25) (layer "B.Cu") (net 20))
 (segment (start 85.09 74.93) (end 78.745 74.93) (width 0.25) (layer "B.Cu") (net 20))
 (segment (start 96.52 106.546682) (end 95.309124 107.757558) (width 0.25) (layer "B.Cu") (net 20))
 (segment (start 96.52 106.546682) (end 96.52 83.494009) (width 0.25) (layer "B.Cu") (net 20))
 (segment (start 91.44 81.28) (end 85.09 74.93) (width 0.25) (layer "B.Cu") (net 20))
 (segment (start 71.12 106.68) (end 72.197558 107.757558) (width 0.25) (layer "B.Cu") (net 20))
 (segment (start 96.52 83.494009) (end 94.305991 81.28) (width 0.25) (layer "B.Cu") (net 20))
 (segment (start 69.945 75.025) (end 72.485 75.025) (width 0.25) (layer "B.Cu") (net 9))
 (segment (start 76.2 78.74) (end 86.36 78.74) (width 0.25) (layer "B.Cu") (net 9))
 (segment (start 68.58 73.66) (end 69.945 75.025) (width 0.25) (layer "B.Cu") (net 9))
 (segment (start 86.36 78.74) (end 92.71 85.09) (width 0.25) (layer "B.Cu") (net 9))
 (segment (start 72.485 75.025) (end 76.2 78.74) (width 0.25) (layer "B.Cu") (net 9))
 (segment (start 92.71 85.09) (end 93.985 85.09) (width 0.25) (layer "B.Cu") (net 9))
 (segment (start 86.492878 57.101524) (end 95.201524 57.101524) (width 0.25) (layer "F.Cu") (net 35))
 (segment (start 95.201524 57.101524) (end 99.06 60.96) (width 0.25) (layer "F.Cu") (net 35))
 (segment (start 90.534945 53.34) (end 91.314513 54.119568) (width 0.25) (layer "F.Cu") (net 33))
 (segment (start 86.36 53.34) (end 90.534945 53.34) (width 0.25) (layer "F.Cu") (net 33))
 (segment (start 96.52 63.5) (end 99.06 66.04) (width 0.25) (layer "B.Cu") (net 34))
 (segment (start 96.52 63.5) (end 96.52 56.785055) (width 0.25) (layer "B.Cu") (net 34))
 (segment (start 96.52 56.785055) (end 93.854513 54.119568) (width 0.25) (layer "B.Cu") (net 34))
 (segment (start 99.06 66.04) (end 99.06 96.52) (width 0.25) (layer "B.Cu") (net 34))
 (segment (start 99.06 96.52) (end 101.6 99.06) (width 0.25) (layer "B.Cu") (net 34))
 (segment (start 86.36 60.96) (end 91.44 60.96) (width 0.25) (layer "F.Cu") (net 36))
 (segment (start 98.080401 98.080401) (end 98.080401 66.501977) (width 0.25) (layer "B.Cu") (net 37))
 (segment (start 93.917107 62.338683) (end 93.98 62.27579) (width 0.25) (layer "B.Cu") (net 37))
 (segment (start 98.080401 66.501977) (end 93.917107 62.338683) (width 0.25) (layer "B.Cu") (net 37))
 (segment (start 101.6 101.6) (end 98.080401 98.080401) (width 0.25) (layer "B.Cu") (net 37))
 (segment (start 93.98 62.27579) (end 93.98 60.96) (width 0.25) (layer "B.Cu") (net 37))
 (segment (start 73.66 73.66) (end 71.12 73.66) (width 0.25) (layer "B.Cu") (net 10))
 (segment (start 76.2 76.2) (end 73.66 73.66) (width 0.25) (layer "B.Cu") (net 10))
 (segment (start 93.985 82.55) (end 91.766504 82.55) (width 0.25) (layer "B.Cu") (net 10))
 (segment (start 91.766504 82.55) (end 85.416504 76.2) (width 0.25) (layer "B.Cu") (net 10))
 (segment (start 85.416504 76.2) (end 76.2 76.2) (width 0.25) (layer "B.Cu") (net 10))
 (segment (start 71.12 71.12) (end 80.83 71.12) (width 0.25) (layer "F.Cu") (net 12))
 (segment (start 80.83 71.12) (end 81.28 71.12) (width 0.25) (layer "F.Cu") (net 12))
 (via (at 81.28 71.12) (size 0.8) (drill 0.4) (layers "F.Cu" "B.Cu") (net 12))
 (segment (start 87.635 71.12) (end 93.985 77.47) (width 0.25) (layer "B.Cu") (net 12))
 (segment (start 81.28 71.12) (end 87.635 71.12) (width 0.25) (layer "B.Cu") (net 12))
 (segment (start 84.95 81.135) (end 93.985 90.17) (width 0.25) (layer "B.Cu") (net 7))
 (segment (start 77.958604 81.135) (end 84.95 81.135) (width 0.25) (layer "B.Cu") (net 7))
 (segment (start 69.945 77.565) (end 74.388604 77.565) (width 0.25) (layer "B.Cu") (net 7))
 (segment (start 68.58 76.2) (end 69.945 77.565) (width 0.25) (layer "B.Cu") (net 7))
 (segment (start 74.388604 77.565) (end 77.958604 81.135) (width 0.25) (layer "B.Cu") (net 7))
 (segment (start 86.494851 87.759852) (end 82.7 83.965) (width 0.25) (layer "B.Cu") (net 5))
 (segment (start 69.945 80.105) (end 68.58 78.74) (width 0.25) (layer "B.Cu") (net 5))
 (segment (start 74.709009 80.105) (end 69.945 80.105) (width 0.25) (layer "B.Cu") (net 5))
 (segment (start 82.7 83.965) (end 78.569009 83.965) (width 0.25) (layer "B.Cu") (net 5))
 (segment (start 86.36 87.625) (end 93.985 95.25) (width 0.25) (layer "B.Cu") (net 5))
 (segment (start 78.569009 83.965) (end 74.709009 80.105) (width 0.25) (layer "B.Cu") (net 5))
 (segment (start 70.39 84.995) (end 77.249009 84.995) (width 0.25) (layer "F.Cu") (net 26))
 (segment (start 80.01 84.764009) (end 80.01 88.905) (width 0.25) (layer "F.Cu") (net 26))
 (segment (start 79.210991 83.965) (end 80.01 84.764009) (width 0.25) (layer "F.Cu") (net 26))
 (segment (start 80.01 88.905) (end 78.745 90.17) (width 0.25) (layer "F.Cu") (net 26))
 (segment (start 68.58 81.28) (end 69.755 82.455) (width 0.25) (layer "F.Cu") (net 26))
 (segment (start 78.279009 83.965) (end 79.210991 83.965) (width 0.25) (layer "F.Cu") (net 26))
 (segment (start 69.755 84.36) (end 70.39 84.995) (width 0.25) (layer "F.Cu") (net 26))
 (segment (start 69.755 82.455) (end 69.755 84.36) (width 0.25) (layer "F.Cu") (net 26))
 (segment (start 77.249009 84.995) (end 78.279009 83.965) (width 0.25) (layer "F.Cu") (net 26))
 (segment (start 81.28 78.74) (end 73.66 78.74) (width 0.25) (layer "F.Cu") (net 8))
 (segment (start 90.17 87.63) (end 81.28 78.74) (width 0.25) (layer "F.Cu") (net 8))
 (segment (start 73.66 78.74) (end 71.12 76.2) (width 0.25) (layer "F.Cu") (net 8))
 (segment (start 93.985 87.63) (end 90.17 87.63) (width 0.25) (layer "F.Cu") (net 8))
 (segment (start 81.163298 90.291702) (end 78.745 92.71) (width 0.25) (layer "F.Cu") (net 27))
 (segment (start 81.163298 87.60778) (end 81.163298 90.291702) (width 0.25) (layer "F.Cu") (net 27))
 (via (at 81.163298 87.60778) (size 0.8) (drill 0.4) (layers "F.Cu" "B.Cu") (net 27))
 (segment (start 80.020433 86.464915) (end 81.163298 87.60778) (width 0.25) (layer "B.Cu") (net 27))
 (segment (start 71.12 81.28) (end 76.304915 86.464915) (width 0.25) (layer "B.Cu") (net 27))
 (segment (start 76.304915 86.464915) (end 79.595941 86.464915) (width 0.25) (layer "B.Cu") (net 27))
 (segment (start 79.595941 86.464915) (end 80.020433 86.464915) (width 0.25) (layer "B.Cu") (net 27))
 (segment (start 73.66 81.28) (end 71.12 78.74) (width 0.25) (layer "F.Cu") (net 6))
 (segment (start 82.555 81.28) (end 73.66 81.28) (width 0.25) (layer "F.Cu") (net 6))
 (segment (start 93.985 92.71) (end 82.555 81.28) (width 0.25) (layer "F.Cu") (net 6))
 (segment (start 73.979577 85.158784) (end 69.918784 85.158784) (width 0.25) (layer "B.Cu") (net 25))
 (segment (start 78.745 87.63) (end 76.450793 87.63) (width 0.25) (layer "B.Cu") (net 25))
 (segment (start 76.450793 87.63) (end 73.979577 85.158784) (width 0.25) (layer "B.Cu") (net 25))
 (segment (start 69.918784 85.158784) (end 68.58 83.82) (width 0.25) (layer "B.Cu") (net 25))
 (segment (start 78.745 82.55) (end 72.39 82.55) (width 0.25) (layer "F.Cu") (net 23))
 (segment (start 72.39 82.55) (end 71.12 83.82) (width 0.25) (layer "F.Cu") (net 23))
 (segment (start 73.66 88.9) (end 73.66 90.165) (width 0.25) (layer "B.Cu") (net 28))
 (segment (start 73.66 90.165) (end 78.745 95.25) (width 0.25) (layer "B.Cu") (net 28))
 (segment (start 72.485 87.725) (end 73.66 88.9) (width 0.25) (layer "B.Cu") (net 28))
 (segment (start 68.58 86.36) (end 69.945 87.725) (width 0.25) (layer "B.Cu") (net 28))
 (segment (start 69.945 87.725) (end 72.485 87.725) (width 0.25) (layer "B.Cu") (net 28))
 (segment (start 73.66 86.36) (end 76.2 88.9) (width 0.25) (layer "B.Cu") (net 4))
 (segment (start 92.71 97.79) (end 93.985 97.79) (width 0.25) (layer "B.Cu") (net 4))
 (segment (start 71.12 86.36) (end 73.66 86.36) (width 0.25) (layer "B.Cu") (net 4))
 (segment (start 83.82 88.9) (end 92.71 97.79) (width 0.25) (layer "B.Cu") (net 4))
 (segment (start 76.2 88.9) (end 83.82 88.9) (width 0.25) (layer "B.Cu") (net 4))
 (segment (start 72.169009 90.265) (end 69.945 90.265) (width 0.25) (layer "B.Cu") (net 3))
 (segment (start 88.995545 96.615544) (end 78.519553 96.615544) (width 0.25) (layer "B.Cu") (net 3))
 (segment (start 92.710001 100.33) (end 88.995545 96.615544) (width 0.25) (layer "B.Cu") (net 3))
 (segment (start 78.519553 96.615544) (end 72.169009 90.265) (width 0.25) (layer "B.Cu") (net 3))
 (segment (start 93.985 100.33) (end 92.710001 100.33) (width 0.25) (layer "B.Cu") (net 3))
 (segment (start 69.945 90.265) (end 68.58 88.9) (width 0.25) (layer "B.Cu") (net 3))
 (segment (start 78.745 97.79) (end 72.295 91.34) (width 0.25) (layer "F.Cu") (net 29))
 (segment (start 72.295 91.34) (end 72.295 90.075) (width 0.25) (layer "F.Cu") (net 29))
 (segment (start 72.295 90.075) (end 71.12 88.9) (width 0.25) (layer "F.Cu") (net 29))
 (segment (start 72.608139 95.010993) (end 72.608139 93.748399) (width 0.25) (layer "B.Cu") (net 30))
 (segment (start 71.65031 92.79057) (end 69.93057 92.79057) (width 0.25) (layer "B.Cu") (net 30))
 (segment (start 72.608139 93.748399) (end 71.65031 92.79057) (width 0.25) (layer "B.Cu") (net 30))
 (segment (start 69.93057 92.79057) (end 68.58 91.44) (width 0.25) (layer "B.Cu") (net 30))
 (segment (start 78.745 100.33) (end 77.927146 100.33) (width 0.25) (layer "B.Cu") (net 30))
 (segment (start 77.927146 100.33) (end 72.608139 95.010993) (width 0.25) (layer "B.Cu") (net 30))
 (segment (start 90.175 99.06) (end 77.956321 99.06) (width 0.25) (layer "B.Cu") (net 2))
 (segment (start 73.939967 94.259967) (end 71.12 91.44) (width 0.25) (layer "B.Cu") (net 2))
 (segment (start 93.985 102.87) (end 90.175 99.06) (width 0.25) (layer "B.Cu") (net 2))
 (segment (start 73.939967 95.043646) (end 73.939967 94.259967) (width 0.25) (layer "B.Cu") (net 2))
 (segment (start 77.956321 99.06) (end 73.939967 95.043646) (width 0.25) (layer "B.Cu") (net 2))
 (segment (start 70.728299 87.63) (end 76.205 87.63) (width 0.25) (layer "F.Cu") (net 24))
 (segment (start 68.58 93.98) (end 69.945 92.615) (width 0.25) (layer "F.Cu") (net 24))
 (segment (start 69.945 88.413299) (end 70.728299 87.63) (width 0.25) (layer "F.Cu") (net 24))
 (segment (start 69.945 92.615) (end 69.945 88.413299) (width 0.25) (layer "F.Cu") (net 24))
 (segment (start 76.205 87.63) (end 78.745 85.09) (width 0.25) (layer "F.Cu") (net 24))
 (segment (start 77.861701 101.6) (end 71.12 94.858299) (width 0.25) (layer "B.Cu") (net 1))
 (segment (start 88.9 101.6) (end 92.71 105.41) (width 0.25) (layer "B.Cu") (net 1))
 (segment (start 71.12 94.858299) (end 71.12 93.98) (width 0.25) (layer "B.Cu") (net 1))
 (segment (start 88.9 101.6) (end 77.861701 101.6) (width 0.25) (layer "B.Cu") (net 1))
 (segment (start 92.71 105.41) (end 93.985 105.41) (width 0.25) (layer "B.Cu") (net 1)))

